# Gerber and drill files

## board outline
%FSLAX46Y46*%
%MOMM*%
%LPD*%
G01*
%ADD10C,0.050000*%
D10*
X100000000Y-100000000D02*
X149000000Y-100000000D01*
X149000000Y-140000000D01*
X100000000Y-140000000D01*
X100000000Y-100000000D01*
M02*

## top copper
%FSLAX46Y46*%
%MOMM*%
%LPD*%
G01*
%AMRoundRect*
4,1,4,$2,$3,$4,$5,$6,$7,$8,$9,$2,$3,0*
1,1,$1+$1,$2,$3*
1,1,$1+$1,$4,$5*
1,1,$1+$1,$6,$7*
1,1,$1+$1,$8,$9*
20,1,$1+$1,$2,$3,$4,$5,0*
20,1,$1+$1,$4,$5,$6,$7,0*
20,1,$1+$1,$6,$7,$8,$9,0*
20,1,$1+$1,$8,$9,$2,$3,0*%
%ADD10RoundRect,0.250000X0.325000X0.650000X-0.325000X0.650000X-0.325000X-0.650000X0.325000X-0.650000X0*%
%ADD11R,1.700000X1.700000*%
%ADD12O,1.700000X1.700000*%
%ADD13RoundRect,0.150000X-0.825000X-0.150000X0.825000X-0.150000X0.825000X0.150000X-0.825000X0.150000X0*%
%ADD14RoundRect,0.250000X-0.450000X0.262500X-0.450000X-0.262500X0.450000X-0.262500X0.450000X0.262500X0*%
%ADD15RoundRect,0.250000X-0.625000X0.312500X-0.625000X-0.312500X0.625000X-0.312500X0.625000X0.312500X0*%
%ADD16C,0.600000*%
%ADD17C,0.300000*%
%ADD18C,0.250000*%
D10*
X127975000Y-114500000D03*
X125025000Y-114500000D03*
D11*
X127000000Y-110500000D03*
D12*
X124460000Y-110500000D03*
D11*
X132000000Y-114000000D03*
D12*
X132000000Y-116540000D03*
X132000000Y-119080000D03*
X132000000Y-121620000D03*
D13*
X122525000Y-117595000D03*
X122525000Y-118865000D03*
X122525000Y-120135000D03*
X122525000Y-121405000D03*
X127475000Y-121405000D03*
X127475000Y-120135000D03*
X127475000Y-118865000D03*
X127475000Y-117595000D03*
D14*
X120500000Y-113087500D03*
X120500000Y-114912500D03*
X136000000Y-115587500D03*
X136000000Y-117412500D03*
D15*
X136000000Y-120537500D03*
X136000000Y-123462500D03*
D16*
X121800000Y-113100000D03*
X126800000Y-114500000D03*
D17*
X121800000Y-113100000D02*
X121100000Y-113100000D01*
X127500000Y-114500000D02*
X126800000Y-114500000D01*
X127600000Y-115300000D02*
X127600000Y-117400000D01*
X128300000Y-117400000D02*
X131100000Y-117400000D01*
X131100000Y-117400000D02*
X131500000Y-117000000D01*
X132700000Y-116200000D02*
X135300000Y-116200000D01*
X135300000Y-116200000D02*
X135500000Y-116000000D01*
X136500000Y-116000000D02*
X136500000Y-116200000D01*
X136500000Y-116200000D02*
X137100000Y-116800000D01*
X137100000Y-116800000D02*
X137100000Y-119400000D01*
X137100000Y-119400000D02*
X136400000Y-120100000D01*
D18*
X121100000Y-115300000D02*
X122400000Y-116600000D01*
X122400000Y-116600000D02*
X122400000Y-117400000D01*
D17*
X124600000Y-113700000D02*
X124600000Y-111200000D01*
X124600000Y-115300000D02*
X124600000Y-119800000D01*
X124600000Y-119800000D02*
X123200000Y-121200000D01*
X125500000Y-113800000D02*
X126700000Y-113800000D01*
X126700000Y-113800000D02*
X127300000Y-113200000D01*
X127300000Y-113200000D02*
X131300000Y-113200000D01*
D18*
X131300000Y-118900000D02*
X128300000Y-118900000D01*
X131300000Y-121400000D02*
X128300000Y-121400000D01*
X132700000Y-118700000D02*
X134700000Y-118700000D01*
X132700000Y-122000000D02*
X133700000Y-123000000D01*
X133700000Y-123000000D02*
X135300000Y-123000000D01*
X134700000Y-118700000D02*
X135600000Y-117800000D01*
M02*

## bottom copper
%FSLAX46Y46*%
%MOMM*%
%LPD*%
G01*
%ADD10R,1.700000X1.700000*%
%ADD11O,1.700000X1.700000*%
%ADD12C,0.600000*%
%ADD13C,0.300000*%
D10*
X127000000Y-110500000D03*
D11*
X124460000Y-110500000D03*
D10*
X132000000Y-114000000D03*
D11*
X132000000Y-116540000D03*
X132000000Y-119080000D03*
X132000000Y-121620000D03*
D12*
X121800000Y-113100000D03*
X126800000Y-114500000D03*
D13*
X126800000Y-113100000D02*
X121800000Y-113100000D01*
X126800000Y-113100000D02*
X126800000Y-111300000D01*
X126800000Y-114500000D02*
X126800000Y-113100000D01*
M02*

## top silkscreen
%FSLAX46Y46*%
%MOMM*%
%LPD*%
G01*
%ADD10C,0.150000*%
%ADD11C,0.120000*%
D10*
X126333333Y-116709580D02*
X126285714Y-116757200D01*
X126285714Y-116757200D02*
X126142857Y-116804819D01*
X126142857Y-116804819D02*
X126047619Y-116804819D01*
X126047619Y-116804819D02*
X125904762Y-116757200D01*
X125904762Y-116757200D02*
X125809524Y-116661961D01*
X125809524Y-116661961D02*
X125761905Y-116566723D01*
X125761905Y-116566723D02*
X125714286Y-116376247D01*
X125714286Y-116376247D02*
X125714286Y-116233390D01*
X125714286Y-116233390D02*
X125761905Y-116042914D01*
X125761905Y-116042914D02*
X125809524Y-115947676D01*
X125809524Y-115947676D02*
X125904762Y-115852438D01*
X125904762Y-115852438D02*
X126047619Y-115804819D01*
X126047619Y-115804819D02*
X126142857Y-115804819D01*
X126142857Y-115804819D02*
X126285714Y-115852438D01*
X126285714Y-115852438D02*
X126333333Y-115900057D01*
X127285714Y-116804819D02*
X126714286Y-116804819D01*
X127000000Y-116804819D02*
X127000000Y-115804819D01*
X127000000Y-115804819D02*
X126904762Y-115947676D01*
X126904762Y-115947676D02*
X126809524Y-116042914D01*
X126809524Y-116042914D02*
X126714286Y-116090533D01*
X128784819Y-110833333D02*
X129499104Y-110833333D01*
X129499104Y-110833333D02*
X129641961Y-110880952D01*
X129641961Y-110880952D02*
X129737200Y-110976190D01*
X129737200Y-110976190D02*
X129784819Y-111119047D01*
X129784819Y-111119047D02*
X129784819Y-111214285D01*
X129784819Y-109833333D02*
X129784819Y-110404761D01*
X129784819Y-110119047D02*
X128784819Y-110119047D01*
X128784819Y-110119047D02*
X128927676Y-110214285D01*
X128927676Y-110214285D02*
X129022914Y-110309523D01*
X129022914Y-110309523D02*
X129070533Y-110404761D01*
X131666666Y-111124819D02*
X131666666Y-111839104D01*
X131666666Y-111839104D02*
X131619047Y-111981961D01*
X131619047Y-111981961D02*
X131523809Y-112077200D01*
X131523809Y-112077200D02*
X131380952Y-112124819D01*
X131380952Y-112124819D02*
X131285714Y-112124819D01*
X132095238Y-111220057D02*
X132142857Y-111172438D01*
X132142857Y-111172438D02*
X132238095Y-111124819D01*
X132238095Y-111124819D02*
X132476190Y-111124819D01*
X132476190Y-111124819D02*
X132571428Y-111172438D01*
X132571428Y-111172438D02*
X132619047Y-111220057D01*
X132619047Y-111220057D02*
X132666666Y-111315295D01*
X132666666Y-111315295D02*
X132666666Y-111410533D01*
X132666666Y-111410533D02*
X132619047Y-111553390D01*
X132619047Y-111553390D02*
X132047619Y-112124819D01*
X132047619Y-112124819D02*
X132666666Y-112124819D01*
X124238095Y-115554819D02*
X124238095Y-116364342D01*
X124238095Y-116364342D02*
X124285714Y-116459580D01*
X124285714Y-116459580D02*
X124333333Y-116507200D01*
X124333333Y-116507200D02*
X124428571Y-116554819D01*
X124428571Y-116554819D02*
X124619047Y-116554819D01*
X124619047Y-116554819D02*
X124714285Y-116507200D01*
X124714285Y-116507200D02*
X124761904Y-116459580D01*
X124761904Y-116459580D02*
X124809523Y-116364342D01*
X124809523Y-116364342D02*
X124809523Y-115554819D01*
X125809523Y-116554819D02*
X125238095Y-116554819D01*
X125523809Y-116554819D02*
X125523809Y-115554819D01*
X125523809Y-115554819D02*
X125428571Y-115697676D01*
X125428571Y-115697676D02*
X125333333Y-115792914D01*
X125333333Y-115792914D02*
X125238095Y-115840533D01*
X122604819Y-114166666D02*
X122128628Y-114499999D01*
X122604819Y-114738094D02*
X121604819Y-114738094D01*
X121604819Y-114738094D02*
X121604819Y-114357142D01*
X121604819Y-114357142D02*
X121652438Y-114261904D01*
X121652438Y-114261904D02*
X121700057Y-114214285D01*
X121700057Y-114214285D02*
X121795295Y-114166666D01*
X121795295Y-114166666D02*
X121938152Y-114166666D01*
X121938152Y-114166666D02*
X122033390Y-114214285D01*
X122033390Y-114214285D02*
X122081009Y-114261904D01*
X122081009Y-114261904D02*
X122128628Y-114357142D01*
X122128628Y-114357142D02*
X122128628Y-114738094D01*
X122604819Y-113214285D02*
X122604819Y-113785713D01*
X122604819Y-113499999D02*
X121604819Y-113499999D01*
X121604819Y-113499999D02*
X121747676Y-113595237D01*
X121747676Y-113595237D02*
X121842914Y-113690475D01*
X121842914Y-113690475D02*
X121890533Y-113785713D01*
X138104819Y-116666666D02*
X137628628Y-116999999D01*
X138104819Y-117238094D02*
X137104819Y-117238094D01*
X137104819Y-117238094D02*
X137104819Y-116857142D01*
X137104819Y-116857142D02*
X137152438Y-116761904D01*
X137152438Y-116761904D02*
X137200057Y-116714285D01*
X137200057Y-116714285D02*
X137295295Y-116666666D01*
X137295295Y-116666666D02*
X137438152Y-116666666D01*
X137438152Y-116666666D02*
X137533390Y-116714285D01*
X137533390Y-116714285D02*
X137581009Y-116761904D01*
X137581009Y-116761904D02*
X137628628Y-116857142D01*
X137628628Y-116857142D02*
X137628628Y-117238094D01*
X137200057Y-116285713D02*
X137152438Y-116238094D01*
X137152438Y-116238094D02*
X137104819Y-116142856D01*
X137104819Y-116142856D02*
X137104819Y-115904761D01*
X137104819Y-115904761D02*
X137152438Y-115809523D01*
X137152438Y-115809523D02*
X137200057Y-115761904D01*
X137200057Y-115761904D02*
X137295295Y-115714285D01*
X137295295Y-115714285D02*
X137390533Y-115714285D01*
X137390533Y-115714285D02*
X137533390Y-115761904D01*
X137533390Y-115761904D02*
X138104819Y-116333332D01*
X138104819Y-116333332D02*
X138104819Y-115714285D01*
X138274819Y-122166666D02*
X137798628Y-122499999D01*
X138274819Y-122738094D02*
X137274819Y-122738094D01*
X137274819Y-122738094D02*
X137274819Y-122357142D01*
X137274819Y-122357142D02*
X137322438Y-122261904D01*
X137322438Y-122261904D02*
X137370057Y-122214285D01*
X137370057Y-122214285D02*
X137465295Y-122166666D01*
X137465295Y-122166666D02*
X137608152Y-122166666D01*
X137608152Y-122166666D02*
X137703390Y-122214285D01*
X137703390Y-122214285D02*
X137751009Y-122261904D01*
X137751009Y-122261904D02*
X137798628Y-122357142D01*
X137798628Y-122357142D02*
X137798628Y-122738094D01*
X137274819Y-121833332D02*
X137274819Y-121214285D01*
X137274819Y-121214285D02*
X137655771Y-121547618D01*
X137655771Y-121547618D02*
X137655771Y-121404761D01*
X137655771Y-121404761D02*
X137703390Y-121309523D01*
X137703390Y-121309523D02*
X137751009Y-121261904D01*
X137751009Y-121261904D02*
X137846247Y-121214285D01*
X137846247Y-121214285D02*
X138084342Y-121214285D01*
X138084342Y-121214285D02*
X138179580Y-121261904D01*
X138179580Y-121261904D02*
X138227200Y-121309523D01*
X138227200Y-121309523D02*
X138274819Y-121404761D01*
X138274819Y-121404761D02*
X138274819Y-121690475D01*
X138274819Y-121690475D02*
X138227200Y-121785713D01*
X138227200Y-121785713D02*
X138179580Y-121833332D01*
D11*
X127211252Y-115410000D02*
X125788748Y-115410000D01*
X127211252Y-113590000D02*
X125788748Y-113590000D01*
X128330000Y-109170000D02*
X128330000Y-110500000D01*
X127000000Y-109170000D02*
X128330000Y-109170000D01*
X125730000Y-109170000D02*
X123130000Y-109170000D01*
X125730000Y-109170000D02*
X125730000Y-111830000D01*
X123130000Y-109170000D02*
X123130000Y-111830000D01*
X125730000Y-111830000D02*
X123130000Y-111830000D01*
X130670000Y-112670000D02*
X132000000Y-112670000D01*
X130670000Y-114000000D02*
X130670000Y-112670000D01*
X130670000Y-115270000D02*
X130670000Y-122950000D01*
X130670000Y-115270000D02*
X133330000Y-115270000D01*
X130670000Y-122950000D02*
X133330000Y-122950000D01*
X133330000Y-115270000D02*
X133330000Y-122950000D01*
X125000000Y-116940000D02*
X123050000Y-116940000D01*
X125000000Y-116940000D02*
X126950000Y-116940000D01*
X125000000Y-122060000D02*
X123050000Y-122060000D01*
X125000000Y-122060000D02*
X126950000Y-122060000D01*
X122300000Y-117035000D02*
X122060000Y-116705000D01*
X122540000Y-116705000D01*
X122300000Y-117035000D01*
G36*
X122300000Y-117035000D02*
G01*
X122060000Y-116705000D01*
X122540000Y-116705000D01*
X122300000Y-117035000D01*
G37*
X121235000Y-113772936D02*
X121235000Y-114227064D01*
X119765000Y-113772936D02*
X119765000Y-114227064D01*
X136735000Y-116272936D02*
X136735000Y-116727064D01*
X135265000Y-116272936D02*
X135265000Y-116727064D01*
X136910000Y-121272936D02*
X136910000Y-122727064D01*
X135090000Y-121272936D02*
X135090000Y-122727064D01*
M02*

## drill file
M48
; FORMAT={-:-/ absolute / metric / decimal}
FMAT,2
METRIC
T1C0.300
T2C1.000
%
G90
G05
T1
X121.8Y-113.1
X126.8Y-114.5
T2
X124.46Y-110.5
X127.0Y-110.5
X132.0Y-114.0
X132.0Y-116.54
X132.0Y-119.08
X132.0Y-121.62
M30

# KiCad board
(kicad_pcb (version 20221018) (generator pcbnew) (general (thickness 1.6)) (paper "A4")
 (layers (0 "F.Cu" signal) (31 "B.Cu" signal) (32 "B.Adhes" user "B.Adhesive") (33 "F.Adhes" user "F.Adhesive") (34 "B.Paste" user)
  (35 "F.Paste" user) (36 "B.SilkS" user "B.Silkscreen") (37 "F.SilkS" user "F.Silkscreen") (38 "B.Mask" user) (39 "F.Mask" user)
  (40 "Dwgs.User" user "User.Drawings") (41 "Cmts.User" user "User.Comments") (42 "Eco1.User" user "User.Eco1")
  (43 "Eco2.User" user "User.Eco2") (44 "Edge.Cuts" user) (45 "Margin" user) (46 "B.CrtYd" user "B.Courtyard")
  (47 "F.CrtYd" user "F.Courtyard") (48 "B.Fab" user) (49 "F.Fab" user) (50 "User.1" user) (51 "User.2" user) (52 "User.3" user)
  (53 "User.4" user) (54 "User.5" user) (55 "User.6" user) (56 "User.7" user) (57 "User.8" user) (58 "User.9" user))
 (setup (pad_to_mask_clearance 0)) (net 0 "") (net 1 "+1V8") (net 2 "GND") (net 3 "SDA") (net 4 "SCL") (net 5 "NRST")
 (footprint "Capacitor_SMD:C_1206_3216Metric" (layer "F.Cu") (at 126.5 114.5 180)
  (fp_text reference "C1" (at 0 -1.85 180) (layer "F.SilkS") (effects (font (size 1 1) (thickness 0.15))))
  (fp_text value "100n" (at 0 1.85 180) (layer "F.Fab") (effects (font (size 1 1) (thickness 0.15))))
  (fp_line (start -0.711252 -0.91) (end 0.711252 -0.91) (stroke (width 0.12) (type solid)) (layer "F.SilkS"))
  (fp_line (start -0.711252 0.91) (end 0.711252 0.91) (stroke (width 0.12) (type solid)) (layer "F.SilkS"))
  (pad "1" smd roundrect (at -1.475 0 180) (size 1.15 1.8) (layers "F.Cu" "F.Paste" "F.Mask") (roundrect_rratio 0.217391) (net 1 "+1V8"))
  (pad "2" smd roundrect (at 1.475 0 180) (size 1.15 1.8) (layers "F.Cu" "F.Paste" "F.Mask") (roundrect_rratio 0.217391) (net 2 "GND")))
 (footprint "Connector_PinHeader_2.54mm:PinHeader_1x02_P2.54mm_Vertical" (layer "F.Cu") (at 127 110.5 -90)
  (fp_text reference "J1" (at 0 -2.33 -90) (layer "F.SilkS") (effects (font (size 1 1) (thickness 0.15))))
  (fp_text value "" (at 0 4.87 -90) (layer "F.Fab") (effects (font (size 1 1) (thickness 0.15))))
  (fp_line (start -1.33 -1.33) (end 0 -1.33) (stroke (width 0.12) (type solid)) (layer "F.SilkS"))
  (fp_line (start -1.33 0) (end -1.33 -1.33) (stroke (width 0.12) (type solid)) (layer "F.SilkS"))
  (fp_line (start -1.33 1.27) (end -1.33 3.87) (stroke (width 0.12) (type solid)) (layer "F.SilkS"))
  (fp_line (start -1.33 1.27) (end 1.33 1.27) (stroke (width 0.12) (type solid)) (layer "F.SilkS"))
  (fp_line (start -1.33 3.87) (end 1.33 3.87) (stroke (width 0.12) (type solid)) (layer "F.SilkS"))
  (fp_line (start 1.33 1.27) (end 1.33 3.87) (stroke (width 0.12) (type solid)) (layer "F.SilkS"))
  (pad "1" thru_hole rect (at 0 0 270) (size 1.7 1.7) (drill 1) (layers "*.Cu" "*.Mask") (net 1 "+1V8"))
  (pad "2" thru_hole oval (at 0 2.54 270) (size 1.7 1.7) (drill 1) (layers "*.Cu" "*.Mask") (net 2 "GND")))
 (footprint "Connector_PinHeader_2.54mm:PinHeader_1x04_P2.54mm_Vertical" (layer "F.Cu") (at 132 114)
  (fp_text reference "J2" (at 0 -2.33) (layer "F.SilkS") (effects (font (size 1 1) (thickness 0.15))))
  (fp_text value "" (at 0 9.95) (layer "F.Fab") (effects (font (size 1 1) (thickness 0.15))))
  (fp_line (start -1.33 -1.33) (end 0 -1.33) (stroke (width 0.12) (type solid)) (layer "F.SilkS"))
  (fp_line (start -1.33 0) (end -1.33 -1.33) (stroke (width 0.12) (type solid)) (layer "F.SilkS"))
  (fp_line (start -1.33 1.27) (end -1.33 8.95) (stroke (width 0.12) (type solid)) (layer "F.SilkS"))
  (fp_line (start -1.33 1.27) (end 1.33 1.27) (stroke (width 0.12) (type solid)) (layer "F.SilkS"))
  (fp_line (start -1.33 8.95) (end 1.33 8.95) (stroke (width 0.12) (type solid)) (layer "F.SilkS"))
  (fp_line (start 1.33 1.27) (end 1.33 8.95) (stroke (width 0.12) (type solid)) (layer "F.SilkS"))
  (pad "1" thru_hole rect (at 0 0) (size 1.7 1.7) (drill 1) (layers "*.Cu" "*.Mask") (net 2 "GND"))
  (pad "2" thru_hole oval (at 0 2.54) (size 1.7 1.7) (drill 1) (layers "*.Cu" "*.Mask") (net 1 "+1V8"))
  (pad "3" thru_hole oval (at 0 5.08) (size 1.7 1.7) (drill 1) (layers "*.Cu" "*.Mask") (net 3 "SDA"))
  (pad "4" thru_hole oval (at 0 7.62) (size 1.7 1.7) (drill 1) (layers "*.Cu" "*.Mask") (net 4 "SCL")))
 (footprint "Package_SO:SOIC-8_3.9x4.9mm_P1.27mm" (layer "F.Cu") (at 125 119.5)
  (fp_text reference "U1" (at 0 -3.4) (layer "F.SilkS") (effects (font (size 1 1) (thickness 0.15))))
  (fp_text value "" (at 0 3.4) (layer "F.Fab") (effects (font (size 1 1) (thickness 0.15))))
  (fp_line (start 0 -2.56) (end -1.95 -2.56) (stroke (width 0.12) (type solid)) (layer "F.SilkS"))
  (fp_line (start 0 -2.56) (end 1.95 -2.56) (stroke (width 0.12) (type solid)) (layer "F.SilkS"))
  (fp_line (start 0 2.56) (end -1.95 2.56) (stroke (width 0.12) (type solid)) (layer "F.SilkS"))
  (fp_line (start 0 2.56) (end 1.95 2.56) (stroke (width 0.12) (type solid)) (layer "F.SilkS"))
  (fp_poly
   (pts (xy -2.7 -2.465) (xy -2.94 -2.795) (xy -2.46 -2.795) (xy -2.7 -2.465)) (stroke (width 0.12) (type solid)) (fill solid)
   (layer "F.SilkS"))
  (pad "1" smd roundrect (at -2.475 -1.905) (size 1.95 0.6) (layers "F.Cu" "F.Paste" "F.Mask") (roundrect_rratio 0.25) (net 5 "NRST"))
  (pad "2" smd roundrect (at -2.475 -0.635) (size 1.95 0.6) (layers "F.Cu" "F.Paste" "F.Mask") (roundrect_rratio 0.25))
  (pad "3" smd roundrect (at -2.475 0.635) (size 1.95 0.6) (layers "F.Cu" "F.Paste" "F.Mask") (roundrect_rratio 0.25))
  (pad "4" smd roundrect (at -2.475 1.905) (size 1.95 0.6) (layers "F.Cu" "F.Paste" "F.Mask") (roundrect_rratio 0.25) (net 2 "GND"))
  (pad "5" smd roundrect (at 2.475 1.905) (size 1.95 0.6) (layers "F.Cu" "F.Paste" "F.Mask") (roundrect_rratio 0.25) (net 4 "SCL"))
  (pad "6" smd roundrect (at 2.475 0.635) (size 1.95 0.6) (layers "F.Cu" "F.Paste" "F.Mask") (roundrect_rratio 0.25))
  (pad "7" smd roundrect (at 2.475 -0.635) (size 1.95 0.6) (layers "F.Cu" "F.Paste" "F.Mask") (roundrect_rratio 0.25) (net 3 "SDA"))
  (pad "8" smd roundrect (at 2.475 -1.905) (size 1.95 0.6) (layers "F.Cu" "F.Paste" "F.Mask") (roundrect_rratio 0.25) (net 1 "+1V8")))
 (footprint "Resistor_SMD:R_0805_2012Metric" (layer "F.Cu") (at 120.5 114 -90)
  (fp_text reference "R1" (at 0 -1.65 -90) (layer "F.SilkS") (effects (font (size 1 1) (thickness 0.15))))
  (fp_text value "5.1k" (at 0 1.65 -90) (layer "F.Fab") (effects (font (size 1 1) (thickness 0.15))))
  (fp_line (start -0.227064 -0.735) (end 0.227064 -0.735) (stroke (width 0.12) (type solid)) (layer "F.SilkS"))
  (fp_line (start -0.227064 0.735) (end 0.227064 0.735) (stroke (width 0.12) (type solid)) (layer "F.SilkS"))
  (pad "1" smd roundrect (at -0.9125 0 270) (size 1.025 1.4) (layers "F.Cu" "F.Paste" "F.Mask") (roundrect_rratio 0.243902) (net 1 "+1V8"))
  (pad "2" smd roundrect (at 0.9125 0 270) (size 1.025 1.4) (layers "F.Cu" "F.Paste" "F.Mask") (roundrect_rratio 0.243902) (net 5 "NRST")))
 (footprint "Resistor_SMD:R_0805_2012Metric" (layer "F.Cu") (at 136 116.5 -90)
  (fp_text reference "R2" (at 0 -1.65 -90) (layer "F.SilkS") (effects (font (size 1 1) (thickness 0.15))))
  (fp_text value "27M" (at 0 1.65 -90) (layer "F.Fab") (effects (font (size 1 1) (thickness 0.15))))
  (fp_line (start -0.227064 -0.735) (end 0.227064 -0.735) (stroke (width 0.12) (type solid)) (layer "F.SilkS"))
  (fp_line (start -0.227064 0.735) (end 0.227064 0.735) (stroke (width 0.12) (type solid)) (layer "F.SilkS"))
  (pad "1" smd roundrect (at -0.9125 0 270) (size 1.025 1.4) (layers "F.Cu" "F.Paste" "F.Mask") (roundrect_rratio 0.243902) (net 1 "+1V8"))
  (pad "2" smd roundrect (at 0.9125 0 270) (size 1.025 1.4) (layers "F.Cu" "F.Paste" "F.Mask") (roundrect_rratio 0.243902) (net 3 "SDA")))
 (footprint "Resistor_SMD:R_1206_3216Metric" (layer "F.Cu") (at 136 122 -90)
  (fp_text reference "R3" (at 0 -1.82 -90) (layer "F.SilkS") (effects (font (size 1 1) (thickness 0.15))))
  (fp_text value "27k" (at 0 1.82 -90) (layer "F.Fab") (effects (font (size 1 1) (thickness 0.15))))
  (fp_line (start -0.727064 -0.91) (end 0.727064 -0.91) (stroke (width 0.12) (type solid)) (layer "F.SilkS"))
  (fp_line (start -0.727064 0.91) (end 0.727064 0.91) (stroke (width 0.12) (type solid)) (layer "F.SilkS"))
  (pad "1" smd roundrect (at -1.4625 0 270) (size 1.125 1.75) (layers "F.Cu" "F.Paste" "F.Mask") (roundrect_rratio 0.222222) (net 1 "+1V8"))
  (pad "2" smd roundrect (at 1.4625 0 270) (size 1.125 1.75) (layers "F.Cu" "F.Paste" "F.Mask") (roundrect_rratio 0.222222) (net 4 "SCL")))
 (gr_rect (start 100 100) (end 149 140) (stroke (width 0.05) (type default)) (fill none) (layer "Edge.Cuts"))
 (segment (start 121.8 113.1) (end 121.1 113.1) (width 0.3) (layer "F.Cu") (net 1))
 (segment (start 127.5 114.5) (end 126.8 114.5) (width 0.3) (layer "F.Cu") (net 1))
 (segment (start 127.6 115.3) (end 127.6 117.4) (width 0.3) (layer "F.Cu") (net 1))
 (segment (start 128.3 117.4) (end 131.1 117.4) (width 0.3) (layer "F.Cu") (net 1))
 (segment (start 131.1 117.4) (end 131.5 117) (width 0.3) (layer "F.Cu") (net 1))
 (segment (start 132.7 116.2) (end 135.3 116.2) (width 0.3) (layer "F.Cu") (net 1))
 (segment (start 135.3 116.2) (end 135.5 116) (width 0.3) (layer "F.Cu") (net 1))
 (segment (start 136.5 116) (end 136.5 116.2) (width 0.3) (layer "F.Cu") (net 1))
 (segment (start 136.5 116.2) (end 137.1 116.8) (width 0.3) (layer "F.Cu") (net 1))
 (segment (start 137.1 116.8) (end 137.1 119.4) (width 0.3) (layer "F.Cu") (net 1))
 (segment (start 137.1 119.4) (end 136.4 120.1) (width 0.3) (layer "F.Cu") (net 1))
 (via (at 121.8 113.1) (size 0.6) (drill 0.3) (layers "F.Cu" "B.Cu") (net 1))
 (via (at 126.8 114.5) (size 0.6) (drill 0.3) (layers "F.Cu" "B.Cu") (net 1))
 (segment (start 121.1 115.3) (end 122.4 116.6) (width 0.25) (layer "F.Cu") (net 5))
 (segment (start 122.4 116.6) (end 122.4 117.4) (width 0.25) (layer "F.Cu") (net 5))
 (segment (start 124.6 113.7) (end 124.6 111.2) (width 0.3) (layer "F.Cu") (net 2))
 (segment (start 124.6 115.3) (end 124.6 119.8) (width 0.3) (layer "F.Cu") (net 2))
 (segment (start 124.6 119.8) (end 123.2 121.2) (width 0.3) (layer "F.Cu") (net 2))
 (segment (start 125.5 113.8) (end 126.7 113.8) (width 0.3) (layer "F.Cu") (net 2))
 (segment (start 126.7 113.8) (end 127.3 113.2) (width 0.3) (layer "F.Cu") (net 2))
 (segment (start 126.8 113.1) (end 121.8 113.1) (width 0.3) (layer "B.Cu") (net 1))
 (segment (start 126.8 113.1) (end 126.8 111.3) (width 0.3) (layer "B.Cu") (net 1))
 (segment (start 126.8 114.5) (end 126.8 113.1) (width 0.3) (layer "B.Cu") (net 1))
 (segment (start 127.3 113.2) (end 131.3 113.2) (width 0.3) (layer "F.Cu") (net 2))
 (segment (start 131.3 118.9) (end 128.3 118.9) (width 0.25) (layer "F.Cu") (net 3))
 (segment (start 131.3 121.4) (end 128.3 121.4) (width 0.25) (layer "F.Cu") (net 4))
 (segment (start 132.7 118.7) (end 134.7 118.7) (width 0.25) (layer "F.Cu") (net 3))
 (segment (start 132.7 122) (end 133.7 123) (width 0.25) (layer "F.Cu") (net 4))
 (segment (start 133.7 123) (end 135.3 123) (width 0.25) (layer "F.Cu") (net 4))
 (segment (start 134.7 118.7) (end 135.6 117.8) (width 0.25) (layer "F.Cu") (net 3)))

